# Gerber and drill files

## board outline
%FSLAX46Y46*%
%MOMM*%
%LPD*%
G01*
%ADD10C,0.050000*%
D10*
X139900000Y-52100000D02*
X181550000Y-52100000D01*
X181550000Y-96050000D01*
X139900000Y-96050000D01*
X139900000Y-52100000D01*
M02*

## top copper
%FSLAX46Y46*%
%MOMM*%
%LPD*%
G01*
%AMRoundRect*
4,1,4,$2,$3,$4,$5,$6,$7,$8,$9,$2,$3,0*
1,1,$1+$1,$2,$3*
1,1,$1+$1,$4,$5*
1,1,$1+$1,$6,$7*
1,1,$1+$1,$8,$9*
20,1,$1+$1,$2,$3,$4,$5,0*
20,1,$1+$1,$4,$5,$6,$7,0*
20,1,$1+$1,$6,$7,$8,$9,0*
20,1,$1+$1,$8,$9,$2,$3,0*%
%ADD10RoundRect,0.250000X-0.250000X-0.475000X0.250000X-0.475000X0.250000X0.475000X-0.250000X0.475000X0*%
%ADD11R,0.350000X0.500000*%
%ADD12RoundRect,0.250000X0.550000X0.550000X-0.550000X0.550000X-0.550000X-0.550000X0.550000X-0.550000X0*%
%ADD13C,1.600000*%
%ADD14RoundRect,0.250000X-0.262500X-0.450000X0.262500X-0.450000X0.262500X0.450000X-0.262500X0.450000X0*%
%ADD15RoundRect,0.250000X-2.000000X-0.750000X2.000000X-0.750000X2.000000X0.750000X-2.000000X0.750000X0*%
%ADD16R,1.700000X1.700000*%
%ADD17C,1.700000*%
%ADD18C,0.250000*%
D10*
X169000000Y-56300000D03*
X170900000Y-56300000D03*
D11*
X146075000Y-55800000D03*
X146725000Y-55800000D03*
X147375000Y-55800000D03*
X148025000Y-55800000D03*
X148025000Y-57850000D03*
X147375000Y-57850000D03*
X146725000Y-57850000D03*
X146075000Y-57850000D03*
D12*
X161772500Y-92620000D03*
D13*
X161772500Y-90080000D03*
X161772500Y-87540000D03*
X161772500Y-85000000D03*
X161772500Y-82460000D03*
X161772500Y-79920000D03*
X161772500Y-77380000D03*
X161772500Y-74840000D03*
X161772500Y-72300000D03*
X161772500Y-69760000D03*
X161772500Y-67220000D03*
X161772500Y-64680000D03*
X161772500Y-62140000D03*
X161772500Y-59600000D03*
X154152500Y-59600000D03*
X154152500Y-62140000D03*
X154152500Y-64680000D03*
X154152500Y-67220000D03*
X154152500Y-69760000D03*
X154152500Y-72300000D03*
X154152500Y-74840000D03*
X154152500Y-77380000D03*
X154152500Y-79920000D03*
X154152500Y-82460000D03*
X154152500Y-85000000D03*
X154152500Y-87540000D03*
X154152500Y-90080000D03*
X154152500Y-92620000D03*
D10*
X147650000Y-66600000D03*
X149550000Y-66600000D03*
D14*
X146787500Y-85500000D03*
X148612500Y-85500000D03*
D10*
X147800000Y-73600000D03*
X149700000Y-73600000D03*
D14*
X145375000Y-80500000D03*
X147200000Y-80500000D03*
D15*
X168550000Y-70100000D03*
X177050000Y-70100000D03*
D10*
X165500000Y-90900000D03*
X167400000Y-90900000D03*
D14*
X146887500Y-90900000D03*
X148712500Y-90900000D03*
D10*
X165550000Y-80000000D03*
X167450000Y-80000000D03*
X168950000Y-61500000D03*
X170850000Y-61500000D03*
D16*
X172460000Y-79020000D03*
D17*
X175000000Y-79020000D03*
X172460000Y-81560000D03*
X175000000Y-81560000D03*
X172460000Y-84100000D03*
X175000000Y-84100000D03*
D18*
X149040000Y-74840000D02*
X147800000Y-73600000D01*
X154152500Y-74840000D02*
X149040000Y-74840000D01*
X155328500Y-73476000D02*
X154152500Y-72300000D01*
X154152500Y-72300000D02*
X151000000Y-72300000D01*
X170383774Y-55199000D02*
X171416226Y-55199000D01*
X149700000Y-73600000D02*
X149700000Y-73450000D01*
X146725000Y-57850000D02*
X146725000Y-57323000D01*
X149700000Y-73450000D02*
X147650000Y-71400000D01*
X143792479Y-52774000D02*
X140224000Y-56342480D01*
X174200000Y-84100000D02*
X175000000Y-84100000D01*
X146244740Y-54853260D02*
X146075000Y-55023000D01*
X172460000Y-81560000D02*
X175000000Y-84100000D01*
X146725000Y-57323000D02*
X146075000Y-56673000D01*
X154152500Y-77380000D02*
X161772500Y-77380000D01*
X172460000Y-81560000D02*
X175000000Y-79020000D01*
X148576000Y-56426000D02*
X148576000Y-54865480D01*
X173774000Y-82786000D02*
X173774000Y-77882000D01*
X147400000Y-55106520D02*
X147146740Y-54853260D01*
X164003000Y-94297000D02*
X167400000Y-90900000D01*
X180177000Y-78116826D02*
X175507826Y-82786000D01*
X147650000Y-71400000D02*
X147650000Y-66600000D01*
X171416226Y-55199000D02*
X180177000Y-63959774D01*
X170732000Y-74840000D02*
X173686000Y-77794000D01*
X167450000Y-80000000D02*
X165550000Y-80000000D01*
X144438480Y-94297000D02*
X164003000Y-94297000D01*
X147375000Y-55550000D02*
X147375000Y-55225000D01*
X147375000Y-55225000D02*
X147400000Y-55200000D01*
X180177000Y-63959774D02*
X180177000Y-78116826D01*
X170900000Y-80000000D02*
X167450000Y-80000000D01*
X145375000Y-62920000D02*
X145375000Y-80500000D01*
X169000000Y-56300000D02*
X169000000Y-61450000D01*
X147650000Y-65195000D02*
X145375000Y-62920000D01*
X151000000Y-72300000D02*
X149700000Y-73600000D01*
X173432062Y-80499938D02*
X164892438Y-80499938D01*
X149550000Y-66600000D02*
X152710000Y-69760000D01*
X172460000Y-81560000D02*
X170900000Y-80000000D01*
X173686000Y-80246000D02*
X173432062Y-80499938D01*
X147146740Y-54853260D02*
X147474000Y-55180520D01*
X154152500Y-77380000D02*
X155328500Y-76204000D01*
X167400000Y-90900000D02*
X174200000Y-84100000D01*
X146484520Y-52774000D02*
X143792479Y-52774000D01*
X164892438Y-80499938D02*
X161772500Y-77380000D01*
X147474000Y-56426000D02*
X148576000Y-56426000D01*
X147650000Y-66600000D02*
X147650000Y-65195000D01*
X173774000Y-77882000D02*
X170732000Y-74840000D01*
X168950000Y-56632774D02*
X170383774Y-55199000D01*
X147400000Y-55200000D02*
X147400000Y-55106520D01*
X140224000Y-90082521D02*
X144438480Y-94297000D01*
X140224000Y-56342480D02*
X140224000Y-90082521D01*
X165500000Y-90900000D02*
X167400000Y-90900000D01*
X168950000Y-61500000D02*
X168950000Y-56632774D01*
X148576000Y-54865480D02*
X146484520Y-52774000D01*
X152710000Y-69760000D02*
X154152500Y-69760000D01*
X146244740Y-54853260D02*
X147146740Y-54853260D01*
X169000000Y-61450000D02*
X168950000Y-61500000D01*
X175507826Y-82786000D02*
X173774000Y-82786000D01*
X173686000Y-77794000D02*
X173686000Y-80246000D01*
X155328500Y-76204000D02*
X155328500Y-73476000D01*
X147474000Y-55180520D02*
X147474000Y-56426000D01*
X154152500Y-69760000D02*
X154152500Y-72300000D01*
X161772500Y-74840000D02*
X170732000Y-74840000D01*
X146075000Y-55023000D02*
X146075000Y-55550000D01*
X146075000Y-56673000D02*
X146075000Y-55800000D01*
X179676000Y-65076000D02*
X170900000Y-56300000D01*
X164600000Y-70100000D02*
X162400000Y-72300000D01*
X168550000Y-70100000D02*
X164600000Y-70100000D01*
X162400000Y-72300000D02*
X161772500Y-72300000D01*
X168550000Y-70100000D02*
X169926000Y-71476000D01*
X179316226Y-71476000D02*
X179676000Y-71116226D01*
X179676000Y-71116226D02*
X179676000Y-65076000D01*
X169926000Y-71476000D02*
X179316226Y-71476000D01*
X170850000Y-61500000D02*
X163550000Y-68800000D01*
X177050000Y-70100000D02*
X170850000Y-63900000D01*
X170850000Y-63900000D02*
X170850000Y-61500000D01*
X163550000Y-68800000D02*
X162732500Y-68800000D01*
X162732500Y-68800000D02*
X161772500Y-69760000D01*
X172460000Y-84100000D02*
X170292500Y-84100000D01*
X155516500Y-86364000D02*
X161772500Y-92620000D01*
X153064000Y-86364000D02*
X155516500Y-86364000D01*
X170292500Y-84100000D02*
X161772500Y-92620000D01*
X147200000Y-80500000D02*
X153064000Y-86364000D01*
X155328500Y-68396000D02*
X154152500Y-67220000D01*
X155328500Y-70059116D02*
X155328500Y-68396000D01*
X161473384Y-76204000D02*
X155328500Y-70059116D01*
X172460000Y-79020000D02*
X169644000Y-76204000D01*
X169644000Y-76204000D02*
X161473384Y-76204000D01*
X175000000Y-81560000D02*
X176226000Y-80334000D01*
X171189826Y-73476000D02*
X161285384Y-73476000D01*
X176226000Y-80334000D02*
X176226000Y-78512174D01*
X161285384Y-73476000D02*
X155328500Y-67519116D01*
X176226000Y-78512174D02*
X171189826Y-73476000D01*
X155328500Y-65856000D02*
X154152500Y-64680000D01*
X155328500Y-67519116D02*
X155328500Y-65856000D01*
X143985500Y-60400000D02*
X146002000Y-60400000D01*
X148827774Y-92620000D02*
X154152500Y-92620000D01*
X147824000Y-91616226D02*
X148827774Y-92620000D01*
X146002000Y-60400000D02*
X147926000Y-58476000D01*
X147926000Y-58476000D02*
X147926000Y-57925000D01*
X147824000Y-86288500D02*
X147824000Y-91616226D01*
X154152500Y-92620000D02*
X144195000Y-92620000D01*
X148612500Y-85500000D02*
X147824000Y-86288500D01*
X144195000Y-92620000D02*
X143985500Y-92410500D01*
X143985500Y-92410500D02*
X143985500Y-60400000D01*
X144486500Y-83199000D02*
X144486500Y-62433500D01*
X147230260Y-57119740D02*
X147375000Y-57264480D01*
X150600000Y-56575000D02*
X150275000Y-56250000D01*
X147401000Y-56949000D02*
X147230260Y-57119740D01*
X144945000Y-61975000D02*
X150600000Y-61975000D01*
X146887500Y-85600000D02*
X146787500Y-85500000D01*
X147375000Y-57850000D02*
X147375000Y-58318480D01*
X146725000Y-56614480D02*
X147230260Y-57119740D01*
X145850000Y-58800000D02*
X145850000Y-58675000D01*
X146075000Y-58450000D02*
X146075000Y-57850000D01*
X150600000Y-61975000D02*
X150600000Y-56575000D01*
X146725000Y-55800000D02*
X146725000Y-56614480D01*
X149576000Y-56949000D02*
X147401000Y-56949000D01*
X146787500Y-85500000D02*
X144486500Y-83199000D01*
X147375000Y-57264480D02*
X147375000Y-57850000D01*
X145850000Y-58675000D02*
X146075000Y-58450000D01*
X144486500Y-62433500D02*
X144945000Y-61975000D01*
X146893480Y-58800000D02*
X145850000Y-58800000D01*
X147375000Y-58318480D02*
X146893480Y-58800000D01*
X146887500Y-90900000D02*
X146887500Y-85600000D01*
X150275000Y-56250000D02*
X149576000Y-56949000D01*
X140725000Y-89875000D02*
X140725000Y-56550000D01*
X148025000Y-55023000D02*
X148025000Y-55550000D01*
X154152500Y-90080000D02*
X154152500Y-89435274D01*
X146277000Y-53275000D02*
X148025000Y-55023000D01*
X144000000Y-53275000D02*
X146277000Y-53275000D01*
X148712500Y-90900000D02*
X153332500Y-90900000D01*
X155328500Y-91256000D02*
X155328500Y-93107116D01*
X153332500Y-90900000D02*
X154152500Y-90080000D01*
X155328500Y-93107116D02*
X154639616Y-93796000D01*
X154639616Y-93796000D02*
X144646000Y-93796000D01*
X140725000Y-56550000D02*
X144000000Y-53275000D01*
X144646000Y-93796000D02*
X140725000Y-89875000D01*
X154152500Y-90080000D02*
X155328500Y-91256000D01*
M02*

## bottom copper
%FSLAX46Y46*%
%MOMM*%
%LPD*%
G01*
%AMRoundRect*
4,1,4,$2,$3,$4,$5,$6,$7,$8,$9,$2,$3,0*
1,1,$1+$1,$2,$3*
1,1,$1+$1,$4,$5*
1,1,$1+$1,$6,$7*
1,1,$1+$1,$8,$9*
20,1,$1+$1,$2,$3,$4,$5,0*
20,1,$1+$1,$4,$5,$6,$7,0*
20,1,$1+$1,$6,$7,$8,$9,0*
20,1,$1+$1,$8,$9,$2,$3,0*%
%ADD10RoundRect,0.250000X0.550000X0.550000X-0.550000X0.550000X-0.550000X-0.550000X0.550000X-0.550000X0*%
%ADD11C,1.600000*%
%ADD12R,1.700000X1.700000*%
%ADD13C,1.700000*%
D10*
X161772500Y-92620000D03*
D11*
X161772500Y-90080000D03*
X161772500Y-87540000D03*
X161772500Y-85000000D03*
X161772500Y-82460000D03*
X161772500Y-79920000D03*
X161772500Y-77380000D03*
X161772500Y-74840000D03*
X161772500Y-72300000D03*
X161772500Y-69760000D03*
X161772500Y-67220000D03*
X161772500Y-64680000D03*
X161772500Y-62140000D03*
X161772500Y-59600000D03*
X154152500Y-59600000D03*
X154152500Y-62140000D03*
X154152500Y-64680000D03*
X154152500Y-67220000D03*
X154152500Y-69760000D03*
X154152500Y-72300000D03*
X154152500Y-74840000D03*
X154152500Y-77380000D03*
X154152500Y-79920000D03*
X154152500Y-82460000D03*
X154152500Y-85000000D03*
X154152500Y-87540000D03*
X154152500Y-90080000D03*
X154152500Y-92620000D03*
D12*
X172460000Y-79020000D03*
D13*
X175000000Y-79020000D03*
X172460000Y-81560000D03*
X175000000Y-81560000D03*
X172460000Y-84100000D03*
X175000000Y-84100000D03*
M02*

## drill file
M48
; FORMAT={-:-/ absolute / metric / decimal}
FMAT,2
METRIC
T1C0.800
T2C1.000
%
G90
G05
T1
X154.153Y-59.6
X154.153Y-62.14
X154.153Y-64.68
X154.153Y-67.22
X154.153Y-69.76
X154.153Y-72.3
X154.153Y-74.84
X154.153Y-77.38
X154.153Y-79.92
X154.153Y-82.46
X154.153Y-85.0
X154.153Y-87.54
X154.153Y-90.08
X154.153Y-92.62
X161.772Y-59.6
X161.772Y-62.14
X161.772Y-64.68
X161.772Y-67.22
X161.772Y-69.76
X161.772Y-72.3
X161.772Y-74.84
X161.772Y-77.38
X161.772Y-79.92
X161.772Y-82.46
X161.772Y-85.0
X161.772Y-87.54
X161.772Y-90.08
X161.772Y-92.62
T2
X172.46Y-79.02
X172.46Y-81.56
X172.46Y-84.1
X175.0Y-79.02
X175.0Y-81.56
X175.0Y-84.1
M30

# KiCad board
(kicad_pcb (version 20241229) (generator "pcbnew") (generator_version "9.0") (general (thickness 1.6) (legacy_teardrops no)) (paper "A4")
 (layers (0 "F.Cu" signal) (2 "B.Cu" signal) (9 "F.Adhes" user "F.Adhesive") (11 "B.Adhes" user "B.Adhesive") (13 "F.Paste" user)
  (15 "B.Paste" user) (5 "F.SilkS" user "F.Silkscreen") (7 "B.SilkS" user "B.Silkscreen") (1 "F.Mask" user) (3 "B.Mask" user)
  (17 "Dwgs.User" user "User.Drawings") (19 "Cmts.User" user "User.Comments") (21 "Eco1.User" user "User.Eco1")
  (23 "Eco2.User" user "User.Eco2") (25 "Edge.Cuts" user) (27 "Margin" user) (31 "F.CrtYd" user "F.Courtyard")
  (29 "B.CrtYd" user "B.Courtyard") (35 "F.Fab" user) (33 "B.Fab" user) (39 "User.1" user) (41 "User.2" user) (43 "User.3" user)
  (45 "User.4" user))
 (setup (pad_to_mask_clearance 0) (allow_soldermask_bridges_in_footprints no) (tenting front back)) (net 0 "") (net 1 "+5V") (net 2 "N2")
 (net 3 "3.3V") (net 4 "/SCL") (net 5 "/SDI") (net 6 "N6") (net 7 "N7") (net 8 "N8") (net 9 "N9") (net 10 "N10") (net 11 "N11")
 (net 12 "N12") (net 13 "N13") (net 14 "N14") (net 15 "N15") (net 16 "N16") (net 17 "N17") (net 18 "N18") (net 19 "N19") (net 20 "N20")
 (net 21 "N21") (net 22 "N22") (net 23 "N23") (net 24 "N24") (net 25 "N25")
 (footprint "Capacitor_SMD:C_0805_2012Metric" (layer "F.Cu") (at 169.95 56.3)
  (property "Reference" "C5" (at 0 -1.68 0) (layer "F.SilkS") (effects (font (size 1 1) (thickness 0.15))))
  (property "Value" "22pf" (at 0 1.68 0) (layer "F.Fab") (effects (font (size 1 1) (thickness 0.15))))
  (pad "1" smd roundrect (at -0.95 0) (size 1 1.45) (layers "F.Cu" "F.Mask" "F.Paste") (roundrect_rratio 0.25) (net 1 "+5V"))
  (pad "2" smd roundrect (at 0.95 0) (size 1 1.45) (layers "F.Cu" "F.Mask" "F.Paste") (roundrect_rratio 0.25) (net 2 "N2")))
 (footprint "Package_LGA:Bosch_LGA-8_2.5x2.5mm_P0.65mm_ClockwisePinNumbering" (layer "F.Cu") (at 147.05 56.825)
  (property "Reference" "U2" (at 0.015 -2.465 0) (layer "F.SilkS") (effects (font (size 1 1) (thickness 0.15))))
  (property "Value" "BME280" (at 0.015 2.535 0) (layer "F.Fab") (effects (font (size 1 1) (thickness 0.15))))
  (pad "1" smd rect (at -0.975 -1.025 90) (size 0.5 0.35) (layers "F.Cu" "F.Mask" "F.Paste") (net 1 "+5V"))
  (pad "2" smd rect (at -0.325 -1.025 90) (size 0.5 0.35) (layers "F.Cu" "F.Mask" "F.Paste") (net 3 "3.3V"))
  (pad "3" smd rect (at 0.325 -1.025 90) (size 0.5 0.35) (layers "F.Cu" "F.Mask" "F.Paste") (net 1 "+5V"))
  (pad "4" smd rect (at 0.975 -1.025 90) (size 0.5 0.35) (layers "F.Cu" "F.Mask" "F.Paste") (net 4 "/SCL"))
  (pad "5" smd rect (at 0.975 1.025 90) (size 0.5 0.35) (layers "F.Cu" "F.Mask" "F.Paste") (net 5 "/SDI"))
  (pad "6" smd rect (at 0.325 1.025 90) (size 0.5 0.35) (layers "F.Cu" "F.Mask" "F.Paste") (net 3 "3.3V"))
  (pad "7" smd rect (at -0.325 1.025 90) (size 0.5 0.35) (layers "F.Cu" "F.Mask" "F.Paste") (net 1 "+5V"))
  (pad "8" smd rect (at -0.975 1.025 90) (size 0.5 0.35) (layers "F.Cu" "F.Mask" "F.Paste") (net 3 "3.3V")))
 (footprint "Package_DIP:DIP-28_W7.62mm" (layer "F.Cu") (at 161.7725 92.62 180)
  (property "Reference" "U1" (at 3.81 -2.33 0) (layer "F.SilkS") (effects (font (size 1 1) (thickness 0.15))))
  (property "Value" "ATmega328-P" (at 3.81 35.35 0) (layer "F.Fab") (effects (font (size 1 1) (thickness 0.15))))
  (pad "1" thru_hole roundrect (at 0 0 180) (size 1.6 1.6) (drill 0.8) (layers "*.Cu" "*.Mask") (remove_unused_layers no)
   (roundrect_rratio 0.15625) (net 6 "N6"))
  (pad "2" thru_hole circle (at 0 2.54 180) (size 1.6 1.6) (drill 0.8) (layers "*.Cu" "*.Mask") (remove_unused_layers no) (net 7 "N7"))
  (pad "3" thru_hole circle (at 0 5.08 180) (size 1.6 1.6) (drill 0.8) (layers "*.Cu" "*.Mask") (remove_unused_layers no) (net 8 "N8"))
  (pad "4" thru_hole circle (at 0 7.62 180) (size 1.6 1.6) (drill 0.8) (layers "*.Cu" "*.Mask") (remove_unused_layers no) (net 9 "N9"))
  (pad "5" thru_hole circle (at 0 10.16 180) (size 1.6 1.6) (drill 0.8) (layers "*.Cu" "*.Mask") (remove_unused_layers no) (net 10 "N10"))
  (pad "6" thru_hole circle (at 0 12.7 180) (size 1.6 1.6) (drill 0.8) (layers "*.Cu" "*.Mask") (remove_unused_layers no) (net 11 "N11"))
  (pad "7" thru_hole circle (at 0 15.24 180) (size 1.6 1.6) (drill 0.8) (layers "*.Cu" "*.Mask") (remove_unused_layers no) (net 1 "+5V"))
  (pad "8" thru_hole circle (at 0 17.78 180) (size 1.6 1.6) (drill 0.8) (layers "*.Cu" "*.Mask") (remove_unused_layers no) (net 1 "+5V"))
  (pad "9" thru_hole circle (at 0 20.32 180) (size 1.6 1.6) (drill 0.8) (layers "*.Cu" "*.Mask") (remove_unused_layers no) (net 2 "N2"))
  (pad "10" thru_hole circle (at 0 22.86 180) (size 1.6 1.6) (drill 0.8) (layers "*.Cu" "*.Mask") (remove_unused_layers no) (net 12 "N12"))
  (pad "11" thru_hole circle (at 0 25.4 180) (size 1.6 1.6) (drill 0.8) (layers "*.Cu" "*.Mask") (remove_unused_layers no) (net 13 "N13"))
  (pad "12" thru_hole circle (at 0 27.94 180) (size 1.6 1.6) (drill 0.8) (layers "*.Cu" "*.Mask") (remove_unused_layers no) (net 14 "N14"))
  (pad "13" thru_hole circle (at 0 30.48 180) (size 1.6 1.6) (drill 0.8) (layers "*.Cu" "*.Mask") (remove_unused_layers no) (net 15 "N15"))
  (pad "14" thru_hole circle (at 0 33.02 180) (size 1.6 1.6) (drill 0.8) (layers "*.Cu" "*.Mask") (remove_unused_layers no) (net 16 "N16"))
  (pad "15" thru_hole circle (at 7.62 33.02 180) (size 1.6 1.6) (drill 0.8) (layers "*.Cu" "*.Mask") (remove_unused_layers no)
   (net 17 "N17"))
  (pad "16" thru_hole circle (at 7.62 30.48 180) (size 1.6 1.6) (drill 0.8) (layers "*.Cu" "*.Mask") (remove_unused_layers no)
   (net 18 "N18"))
  (pad "17" thru_hole circle (at 7.62 27.94 180) (size 1.6 1.6) (drill 0.8) (layers "*.Cu" "*.Mask") (remove_unused_layers no)
   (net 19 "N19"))
  (pad "18" thru_hole circle (at 7.62 25.4 180) (size 1.6 1.6) (drill 0.8) (layers "*.Cu" "*.Mask") (remove_unused_layers no) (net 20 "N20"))
  (pad "19" thru_hole circle (at 7.62 22.86 180) (size 1.6 1.6) (drill 0.8) (layers "*.Cu" "*.Mask") (remove_unused_layers no) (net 1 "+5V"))
  (pad "20" thru_hole circle (at 7.62 20.32 180) (size 1.6 1.6) (drill 0.8) (layers "*.Cu" "*.Mask") (remove_unused_layers no) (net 1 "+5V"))
  (pad "21" thru_hole circle (at 7.62 17.78 180) (size 1.6 1.6) (drill 0.8) (layers "*.Cu" "*.Mask") (remove_unused_layers no)
   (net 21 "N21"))
  (pad "22" thru_hole circle (at 7.62 15.24 180) (size 1.6 1.6) (drill 0.8) (layers "*.Cu" "*.Mask") (remove_unused_layers no) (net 1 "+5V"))
  (pad "23" thru_hole circle (at 7.62 12.7 180) (size 1.6 1.6) (drill 0.8) (layers "*.Cu" "*.Mask") (remove_unused_layers no) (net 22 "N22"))
  (pad "24" thru_hole circle (at 7.62 10.16 180) (size 1.6 1.6) (drill 0.8) (layers "*.Cu" "*.Mask") (remove_unused_layers no)
   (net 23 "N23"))
  (pad "25" thru_hole circle (at 7.62 7.62 180) (size 1.6 1.6) (drill 0.8) (layers "*.Cu" "*.Mask") (remove_unused_layers no) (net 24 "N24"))
  (pad "26" thru_hole circle (at 7.62 5.08 180) (size 1.6 1.6) (drill 0.8) (layers "*.Cu" "*.Mask") (remove_unused_layers no) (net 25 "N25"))
  (pad "27" thru_hole circle (at 7.62 2.54 180) (size 1.6 1.6) (drill 0.8) (layers "*.Cu" "*.Mask") (remove_unused_layers no) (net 4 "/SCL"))
  (pad "28" thru_hole circle (at 7.62 0 180) (size 1.6 1.6) (drill 0.8) (layers "*.Cu" "*.Mask") (remove_unused_layers no) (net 5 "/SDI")))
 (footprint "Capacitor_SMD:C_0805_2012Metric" (layer "F.Cu") (at 148.6 66.6)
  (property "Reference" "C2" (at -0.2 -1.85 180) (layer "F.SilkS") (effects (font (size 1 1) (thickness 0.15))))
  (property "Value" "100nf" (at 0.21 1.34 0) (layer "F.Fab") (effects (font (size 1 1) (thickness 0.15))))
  (pad "1" smd roundrect (at -0.95 0) (size 1 1.45) (layers "F.Cu" "F.Mask" "F.Paste") (roundrect_rratio 0.25) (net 1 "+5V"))
  (pad "2" smd roundrect (at 0.95 0) (size 1 1.45) (layers "F.Cu" "F.Mask" "F.Paste") (roundrect_rratio 0.25) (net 1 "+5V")))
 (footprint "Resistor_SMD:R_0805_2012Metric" (layer "F.Cu") (at 147.7 85.5)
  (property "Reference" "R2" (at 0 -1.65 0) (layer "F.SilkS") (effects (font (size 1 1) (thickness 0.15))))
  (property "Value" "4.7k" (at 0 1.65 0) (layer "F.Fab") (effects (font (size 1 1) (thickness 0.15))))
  (pad "1" smd roundrect (at -0.9125 0) (size 1.025 1.4) (layers "F.Cu" "F.Mask" "F.Paste") (roundrect_rratio 0.243902) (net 3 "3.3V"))
  (pad "2" smd roundrect (at 0.9125 0) (size 1.025 1.4) (layers "F.Cu" "F.Mask" "F.Paste") (roundrect_rratio 0.243902) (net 5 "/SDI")))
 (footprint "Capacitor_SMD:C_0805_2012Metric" (layer "F.Cu") (at 148.75 73.6)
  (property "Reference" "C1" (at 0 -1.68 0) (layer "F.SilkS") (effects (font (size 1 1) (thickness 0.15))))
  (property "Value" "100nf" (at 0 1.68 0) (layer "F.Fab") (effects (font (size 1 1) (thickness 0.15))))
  (pad "1" smd roundrect (at -0.95 0) (size 1 1.45) (layers "F.Cu" "F.Mask" "F.Paste") (roundrect_rratio 0.25) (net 21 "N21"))
  (pad "2" smd roundrect (at 0.95 0) (size 1 1.45) (layers "F.Cu" "F.Mask" "F.Paste") (roundrect_rratio 0.25) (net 1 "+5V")))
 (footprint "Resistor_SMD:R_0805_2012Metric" (layer "F.Cu") (at 146.2875 80.5)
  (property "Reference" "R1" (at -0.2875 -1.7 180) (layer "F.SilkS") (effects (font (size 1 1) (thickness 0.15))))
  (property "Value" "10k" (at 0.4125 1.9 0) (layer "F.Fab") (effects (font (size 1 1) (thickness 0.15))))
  (pad "1" smd roundrect (at -0.9125 0) (size 1.025 1.4) (layers "F.Cu" "F.Mask" "F.Paste") (roundrect_rratio 0.243902) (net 1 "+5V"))
  (pad "2" smd roundrect (at 0.9125 0) (size 1.025 1.4) (layers "F.Cu" "F.Mask" "F.Paste") (roundrect_rratio 0.243902) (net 6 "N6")))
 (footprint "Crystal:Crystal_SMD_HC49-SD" (layer "F.Cu") (at 172.8 70.1)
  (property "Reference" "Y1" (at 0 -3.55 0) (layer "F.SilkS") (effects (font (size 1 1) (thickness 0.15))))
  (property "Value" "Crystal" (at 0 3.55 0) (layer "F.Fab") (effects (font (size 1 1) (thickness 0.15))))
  (pad "1" smd roundrect (at -4.25 0) (size 4.5 2) (layers "F.Cu" "F.Mask" "F.Paste") (roundrect_rratio 0.125) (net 2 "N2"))
  (pad "2" smd roundrect (at 4.25 0) (size 4.5 2) (layers "F.Cu" "F.Mask" "F.Paste") (roundrect_rratio 0.125) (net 12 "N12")))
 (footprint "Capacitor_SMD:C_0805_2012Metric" (layer "F.Cu") (at 166.45 90.9)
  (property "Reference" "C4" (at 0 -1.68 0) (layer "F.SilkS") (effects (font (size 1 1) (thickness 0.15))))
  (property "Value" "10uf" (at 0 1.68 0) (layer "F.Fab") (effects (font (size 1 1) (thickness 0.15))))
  (pad "1" smd roundrect (at -0.95 0) (size 1 1.45) (layers "F.Cu" "F.Mask" "F.Paste") (roundrect_rratio 0.25) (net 1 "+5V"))
  (pad "2" smd roundrect (at 0.95 0) (size 1 1.45) (layers "F.Cu" "F.Mask" "F.Paste") (roundrect_rratio 0.25) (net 1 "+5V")))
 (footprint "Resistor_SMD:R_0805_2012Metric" (layer "F.Cu") (at 147.8 90.9)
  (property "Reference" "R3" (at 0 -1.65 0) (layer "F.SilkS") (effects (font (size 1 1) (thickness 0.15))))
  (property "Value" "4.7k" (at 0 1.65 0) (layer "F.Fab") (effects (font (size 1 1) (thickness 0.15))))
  (pad "1" smd roundrect (at -0.9125 0) (size 1.025 1.4) (layers "F.Cu" "F.Mask" "F.Paste") (roundrect_rratio 0.243902) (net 3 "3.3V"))
  (pad "2" smd roundrect (at 0.9125 0) (size 1.025 1.4) (layers "F.Cu" "F.Mask" "F.Paste") (roundrect_rratio 0.243902) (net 4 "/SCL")))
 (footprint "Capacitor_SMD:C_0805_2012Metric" (layer "F.Cu") (at 166.5 80)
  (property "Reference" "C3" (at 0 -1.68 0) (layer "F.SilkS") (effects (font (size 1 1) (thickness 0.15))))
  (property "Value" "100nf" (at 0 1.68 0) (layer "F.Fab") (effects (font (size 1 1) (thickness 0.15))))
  (pad "1" smd roundrect (at -0.95 0) (size 1 1.45) (layers "F.Cu" "F.Mask" "F.Paste") (roundrect_rratio 0.25) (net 1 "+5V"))
  (pad "2" smd roundrect (at 0.95 0) (size 1 1.45) (layers "F.Cu" "F.Mask" "F.Paste") (roundrect_rratio 0.25) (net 1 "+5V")))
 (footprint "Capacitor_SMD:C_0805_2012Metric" (layer "F.Cu") (at 169.9 61.5)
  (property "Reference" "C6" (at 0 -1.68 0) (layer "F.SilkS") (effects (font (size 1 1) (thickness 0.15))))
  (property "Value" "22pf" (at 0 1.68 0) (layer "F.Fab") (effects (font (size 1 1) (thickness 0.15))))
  (pad "1" smd roundrect (at -0.95 0) (size 1 1.45) (layers "F.Cu" "F.Mask" "F.Paste") (roundrect_rratio 0.25) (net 1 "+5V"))
  (pad "2" smd roundrect (at 0.95 0) (size 1 1.45) (layers "F.Cu" "F.Mask" "F.Paste") (roundrect_rratio 0.25) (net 12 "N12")))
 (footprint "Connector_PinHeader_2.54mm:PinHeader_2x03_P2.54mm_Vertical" (layer "F.Cu") (at 172.46 79.02)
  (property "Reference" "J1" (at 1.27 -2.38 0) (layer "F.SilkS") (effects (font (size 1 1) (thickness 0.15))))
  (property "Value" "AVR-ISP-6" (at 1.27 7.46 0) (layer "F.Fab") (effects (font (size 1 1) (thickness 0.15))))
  (pad "1" thru_hole rect (at 0 0) (size 1.7 1.7) (drill 1) (layers "*.Cu" "*.Mask") (remove_unused_layers no) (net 20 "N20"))
  (pad "2" thru_hole circle (at 2.54 0) (size 1.7 1.7) (drill 1) (layers "*.Cu" "*.Mask") (remove_unused_layers no) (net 1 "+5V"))
  (pad "3" thru_hole circle (at 0 2.54) (size 1.7 1.7) (drill 1) (layers "*.Cu" "*.Mask") (remove_unused_layers no) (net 1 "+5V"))
  (pad "4" thru_hole circle (at 2.54 2.54) (size 1.7 1.7) (drill 1) (layers "*.Cu" "*.Mask") (remove_unused_layers no) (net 19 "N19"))
  (pad "5" thru_hole circle (at 0 5.08) (size 1.7 1.7) (drill 1) (layers "*.Cu" "*.Mask") (remove_unused_layers no) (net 6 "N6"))
  (pad "6" thru_hole circle (at 2.54 5.08) (size 1.7 1.7) (drill 1) (layers "*.Cu" "*.Mask") (remove_unused_layers no) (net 1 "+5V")))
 (gr_rect (start 139.9 52.1) (end 181.55 96.05) (stroke (width 0.05) (type default)) (fill no) (layer "Edge.Cuts"))
 (segment (start 149.04 74.84) (end 147.8 73.6) (width 0.25) (layer "F.Cu") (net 21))
 (segment (start 154.1525 74.84) (end 149.04 74.84) (width 0.25) (layer "F.Cu") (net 21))
 (segment (start 155.3285 73.476) (end 154.1525 72.3) (width 0.25) (layer "F.Cu") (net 1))
 (segment (start 154.1525 72.3) (end 151 72.3) (width 0.25) (layer "F.Cu") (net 1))
 (segment (start 170.383774 55.199) (end 171.416226 55.199) (width 0.25) (layer "F.Cu") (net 1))
 (segment (start 149.7 73.6) (end 149.7 73.45) (width 0.25) (layer "F.Cu") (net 1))
 (segment (start 146.725 57.85) (end 146.725 57.323) (width 0.25) (layer "F.Cu") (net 1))
 (segment (start 149.7 73.45) (end 147.65 71.4) (width 0.25) (layer "F.Cu") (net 1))
 (segment (start 143.792479 52.774) (end 140.224 56.34248) (width 0.25) (layer "F.Cu") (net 1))
 (segment (start 174.2 84.1) (end 175 84.1) (width 0.25) (layer "F.Cu") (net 1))
 (segment (start 146.24474 54.85326) (end 146.075 55.023) (width 0.25) (layer "F.Cu") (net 1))
 (segment (start 172.46 81.56) (end 175 84.1) (width 0.25) (layer "F.Cu") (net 1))
 (segment (start 146.725 57.323) (end 146.075 56.673) (width 0.25) (layer "F.Cu") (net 1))
 (segment (start 154.1525 77.38) (end 161.7725 77.38) (width 0.25) (layer "F.Cu") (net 1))
 (segment (start 172.46 81.56) (end 175 79.02) (width 0.25) (layer "F.Cu") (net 1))
 (segment (start 148.576 56.426) (end 148.576 54.86548) (width 0.25) (layer "F.Cu") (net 1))
 (segment (start 173.774 82.786) (end 173.774 77.882) (width 0.25) (layer "F.Cu") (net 1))
 (segment (start 147.4 55.10652) (end 147.14674 54.85326) (width 0.25) (layer "F.Cu") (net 1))
 (segment (start 164.003 94.297) (end 167.4 90.9) (width 0.25) (layer "F.Cu") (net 1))
 (segment (start 180.177 78.116826) (end 175.507826 82.786) (width 0.25) (layer "F.Cu") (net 1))
 (segment (start 147.65 71.4) (end 147.65 66.6) (width 0.25) (layer "F.Cu") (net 1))
 (segment (start 171.416226 55.199) (end 180.177 63.959774) (width 0.25) (layer "F.Cu") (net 1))
 (segment (start 170.732 74.84) (end 173.686 77.794) (width 0.25) (layer "F.Cu") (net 1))
 (segment (start 167.45 80) (end 165.55 80) (width 0.25) (layer "F.Cu") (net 1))
 (segment (start 144.43848 94.297) (end 164.003 94.297) (width 0.25) (layer "F.Cu") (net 1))
 (segment (start 147.375 55.55) (end 147.375 55.225) (width 0.25) (layer "F.Cu") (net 1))
 (segment (start 147.375 55.225) (end 147.4 55.2) (width 0.25) (layer "F.Cu") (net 1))
 (segment (start 180.177 63.959774) (end 180.177 78.116826) (width 0.25) (layer "F.Cu") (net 1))
 (segment (start 170.9 80) (end 167.45 80) (width 0.25) (layer "F.Cu") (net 1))
 (segment (start 145.375 62.92) (end 145.375 80.5) (width 0.25) (layer "F.Cu") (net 1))
 (segment (start 169 56.3) (end 169 61.45) (width 0.25) (layer "F.Cu") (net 1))
 (segment (start 147.65 65.195) (end 145.375 62.92) (width 0.25) (layer "F.Cu") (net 1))
 (segment (start 151 72.3) (end 149.7 73.6) (width 0.25) (layer "F.Cu") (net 1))
 (segment (start 173.432062 80.499938) (end 164.892438 80.499938) (width 0.25) (layer "F.Cu") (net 1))
 (segment (start 149.55 66.6) (end 152.71 69.76) (width 0.25) (layer "F.Cu") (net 1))
 (segment (start 172.46 81.56) (end 170.9 80) (width 0.25) (layer "F.Cu") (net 1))
 (segment (start 173.686 80.246) (end 173.432062 80.499938) (width 0.25) (layer "F.Cu") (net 1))
 (segment (start 147.14674 54.85326) (end 147.474 55.18052) (width 0.25) (layer "F.Cu") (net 1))
 (segment (start 154.1525 77.38) (end 155.3285 76.204) (width 0.25) (layer "F.Cu") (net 1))
 (segment (start 167.4 90.9) (end 174.2 84.1) (width 0.25) (layer "F.Cu") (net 1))
 (segment (start 146.48452 52.774) (end 143.792479 52.774) (width 0.25) (layer "F.Cu") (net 1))
 (segment (start 164.892438 80.499938) (end 161.7725 77.38) (width 0.25) (layer "F.Cu") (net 1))
 (segment (start 147.474 56.426) (end 148.576 56.426) (width 0.25) (layer "F.Cu") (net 1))
 (segment (start 147.65 66.6) (end 147.65 65.195) (width 0.25) (layer "F.Cu") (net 1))
 (segment (start 173.774 77.882) (end 170.732 74.84) (width 0.25) (layer "F.Cu") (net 1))
 (segment (start 168.95 56.632774) (end 170.383774 55.199) (width 0.25) (layer "F.Cu") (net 1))
 (segment (start 147.4 55.2) (end 147.4 55.10652) (width 0.25) (layer "F.Cu") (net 1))
 (segment (start 140.224 90.082521) (end 144.43848 94.297) (width 0.25) (layer "F.Cu") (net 1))
 (segment (start 140.224 56.34248) (end 140.224 90.082521) (width 0.25) (layer "F.Cu") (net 1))
 (segment (start 165.5 90.9) (end 167.4 90.9) (width 0.25) (layer "F.Cu") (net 1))
 (segment (start 168.95 61.5) (end 168.95 56.632774) (width 0.25) (layer "F.Cu") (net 1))
 (segment (start 148.576 54.86548) (end 146.48452 52.774) (width 0.25) (layer "F.Cu") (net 1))
 (segment (start 152.71 69.76) (end 154.1525 69.76) (width 0.25) (layer "F.Cu") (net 1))
 (segment (start 146.24474 54.85326) (end 147.14674 54.85326) (width 0.25) (layer "F.Cu") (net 1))
 (segment (start 169 61.45) (end 168.95 61.5) (width 0.25) (layer "F.Cu") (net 1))
 (segment (start 175.507826 82.786) (end 173.774 82.786) (width 0.25) (layer "F.Cu") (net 1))
 (segment (start 173.686 77.794) (end 173.686 80.246) (width 0.25) (layer "F.Cu") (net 1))
 (segment (start 155.3285 76.204) (end 155.3285 73.476) (width 0.25) (layer "F.Cu") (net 1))
 (segment (start 147.474 55.18052) (end 147.474 56.426) (width 0.25) (layer "F.Cu") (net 1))
 (segment (start 154.1525 69.76) (end 154.1525 72.3) (width 0.25) (layer "F.Cu") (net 1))
 (segment (start 161.7725 74.84) (end 170.732 74.84) (width 0.25) (layer "F.Cu") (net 1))
 (segment (start 146.075 55.023) (end 146.075 55.55) (width 0.25) (layer "F.Cu") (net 1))
 (segment (start 146.075 56.673) (end 146.075 55.8) (width 0.25) (layer "F.Cu") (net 1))
 (segment (start 179.676 65.076) (end 170.9 56.3) (width 0.25) (layer "F.Cu") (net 2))
 (segment (start 164.6 70.1) (end 162.4 72.3) (width 0.25) (layer "F.Cu") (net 2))
 (segment (start 168.55 70.1) (end 164.6 70.1) (width 0.25) (layer "F.Cu") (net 2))
 (segment (start 162.4 72.3) (end 161.7725 72.3) (width 0.25) (layer "F.Cu") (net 2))
 (segment (start 168.55 70.1) (end 169.926 71.476) (width 0.25) (layer "F.Cu") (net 2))
 (segment (start 179.316226 71.476) (end 179.676 71.116226) (width 0.25) (layer "F.Cu") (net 2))
 (segment (start 179.676 71.116226) (end 179.676 65.076) (width 0.25) (layer "F.Cu") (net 2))
 (segment (start 169.926 71.476) (end 179.316226 71.476) (width 0.25) (layer "F.Cu") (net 2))
 (segment (start 170.85 61.5) (end 163.55 68.8) (width 0.25) (layer "F.Cu") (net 12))
 (segment (start 177.05 70.1) (end 170.85 63.9) (width 0.25) (layer "F.Cu") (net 12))
 (segment (start 170.85 63.9) (end 170.85 61.5) (width 0.25) (layer "F.Cu") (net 12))
 (segment (start 163.55 68.8) (end 162.7325 68.8) (width 0.25) (layer "F.Cu") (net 12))
 (segment (start 162.7325 68.8) (end 161.7725 69.76) (width 0.25) (layer "F.Cu") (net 12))
 (segment (start 172.46 84.1) (end 170.2925 84.1) (width 0.25) (layer "F.Cu") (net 6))
 (segment (start 155.5165 86.364) (end 161.7725 92.62) (width 0.25) (layer "F.Cu") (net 6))
 (segment (start 153.064 86.364) (end 155.5165 86.364) (width 0.25) (layer "F.Cu") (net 6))
 (segment (start 170.2925 84.1) (end 161.7725 92.62) (width 0.25) (layer "F.Cu") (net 6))
 (segment (start 147.2 80.5) (end 153.064 86.364) (width 0.25) (layer "F.Cu") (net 6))
 (segment (start 155.3285 68.396) (end 154.1525 67.22) (width 0.25) (layer "F.Cu") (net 20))
 (segment (start 155.3285 70.059116) (end 155.3285 68.396) (width 0.25) (layer "F.Cu") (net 20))
 (segment (start 161.473384 76.204) (end 155.3285 70.059116) (width 0.25) (layer "F.Cu") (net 20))
 (segment (start 172.46 79.02) (end 169.644 76.204) (width 0.25) (layer "F.Cu") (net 20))
 (segment (start 169.644 76.204) (end 161.473384 76.204) (width 0.25) (layer "F.Cu") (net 20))
 (segment (start 175 81.56) (end 176.226 80.334) (width 0.25) (layer "F.Cu") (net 19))
 (segment (start 171.189826 73.476) (end 161.285384 73.476) (width 0.25) (layer "F.Cu") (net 19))
 (segment (start 176.226 80.334) (end 176.226 78.512174) (width 0.25) (layer "F.Cu") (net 19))
 (segment (start 161.285384 73.476) (end 155.3285 67.519116) (width 0.25) (layer "F.Cu") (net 19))
 (segment (start 176.226 78.512174) (end 171.189826 73.476) (width 0.25) (layer "F.Cu") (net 19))
 (segment (start 155.3285 65.856) (end 154.1525 64.68) (width 0.25) (layer "F.Cu") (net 19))
 (segment (start 155.3285 67.519116) (end 155.3285 65.856) (width 0.25) (layer "F.Cu") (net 19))
 (segment (start 143.9855 60.4) (end 146.002 60.4) (width 0.25) (layer "F.Cu") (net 5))
 (segment (start 148.827774 92.62) (end 154.1525 92.62) (width 0.25) (layer "F.Cu") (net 5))
 (segment (start 147.824 91.616226) (end 148.827774 92.62) (width 0.25) (layer "F.Cu") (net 5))
 (segment (start 146.002 60.4) (end 147.926 58.476) (width 0.25) (layer "F.Cu") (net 5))
 (segment (start 147.926 58.476) (end 147.926 57.925) (width 0.25) (layer "F.Cu") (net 5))
 (segment (start 147.824 86.2885) (end 147.824 91.616226) (width 0.25) (layer "F.Cu") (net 5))
 (segment (start 154.1525 92.62) (end 144.195 92.62) (width 0.25) (layer "F.Cu") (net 5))
 (segment (start 148.6125 85.5) (end 147.824 86.2885) (width 0.25) (layer "F.Cu") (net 5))
 (segment (start 144.195 92.62) (end 143.9855 92.4105) (width 0.25) (layer "F.Cu") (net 5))
 (segment (start 143.9855 92.4105) (end 143.9855 60.4) (width 0.25) (layer "F.Cu") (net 5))
 (segment (start 144.4865 83.199) (end 144.4865 62.4335) (width 0.25) (layer "F.Cu") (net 3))
 (segment (start 147.23026 57.11974) (end 147.375 57.26448) (width 0.25) (layer "F.Cu") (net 3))
 (segment (start 150.6 56.575) (end 150.275 56.25) (width 0.25) (layer "F.Cu") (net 3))
 (segment (start 147.401 56.949) (end 147.23026 57.11974) (width 0.25) (layer "F.Cu") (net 3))
 (segment (start 144.945 61.975) (end 150.6 61.975) (width 0.25) (layer "F.Cu") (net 3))
 (segment (start 146.8875 85.6) (end 146.7875 85.5) (width 0.25) (layer "F.Cu") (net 3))
 (segment (start 147.375 57.85) (end 147.375 58.31848) (width 0.25) (layer "F.Cu") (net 3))
 (segment (start 146.725 56.61448) (end 147.23026 57.11974) (width 0.25) (layer "F.Cu") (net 3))
 (segment (start 145.85 58.8) (end 145.85 58.675) (width 0.25) (layer "F.Cu") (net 3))
 (segment (start 146.075 58.45) (end 146.075 57.85) (width 0.25) (layer "F.Cu") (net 3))
 (segment (start 150.6 61.975) (end 150.6 56.575) (width 0.25) (layer "F.Cu") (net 3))
 (segment (start 146.725 55.8) (end 146.725 56.61448) (width 0.25) (layer "F.Cu") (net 3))
 (segment (start 149.576 56.949) (end 147.401 56.949) (width 0.25) (layer "F.Cu") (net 3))
 (segment (start 146.7875 85.5) (end 144.4865 83.199) (width 0.25) (layer "F.Cu") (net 3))
 (segment (start 147.375 57.26448) (end 147.375 57.85) (width 0.25) (layer "F.Cu") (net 3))
 (segment (start 145.85 58.675) (end 146.075 58.45) (width 0.25) (layer "F.Cu") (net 3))
 (segment (start 144.4865 62.4335) (end 144.945 61.975) (width 0.25) (layer "F.Cu") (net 3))
 (segment (start 146.89348 58.8) (end 145.85 58.8) (width 0.25) (layer "F.Cu") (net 3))
 (segment (start 147.375 58.31848) (end 146.89348 58.8) (width 0.25) (layer "F.Cu") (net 3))
 (segment (start 146.8875 90.9) (end 146.8875 85.6) (width 0.25) (layer "F.Cu") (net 3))
 (segment (start 150.275 56.25) (end 149.576 56.949) (width 0.25) (layer "F.Cu") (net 3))
 (segment (start 140.725 89.875) (end 140.725 56.55) (width 0.25) (layer "F.Cu") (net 4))
 (segment (start 148.025 55.023) (end 148.025 55.55) (width 0.25) (layer "F.Cu") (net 4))
 (segment (start 154.1525 90.08) (end 154.1525 89.435274) (width 0.25) (layer "F.Cu") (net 4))
 (segment (start 146.277 53.275) (end 148.025 55.023) (width 0.25) (layer "F.Cu") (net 4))
 (segment (start 144 53.275) (end 146.277 53.275) (width 0.25) (layer "F.Cu") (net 4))
 (segment (start 148.7125 90.9) (end 153.3325 90.9) (width 0.25) (layer "F.Cu") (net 4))
 (segment (start 155.3285 91.256) (end 155.3285 93.107116) (width 0.25) (layer "F.Cu") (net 4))
 (segment (start 153.3325 90.9) (end 154.1525 90.08) (width 0.25) (layer "F.Cu") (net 4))
 (segment (start 155.3285 93.107116) (end 154.639616 93.796) (width 0.25) (layer "F.Cu") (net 4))
 (segment (start 154.639616 93.796) (end 144.646 93.796) (width 0.25) (layer "F.Cu") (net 4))
 (segment (start 140.725 56.55) (end 144 53.275) (width 0.25) (layer "F.Cu") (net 4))
 (segment (start 144.646 93.796) (end 140.725 89.875) (width 0.25) (layer "F.Cu") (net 4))
 (segment (start 154.1525 90.08) (end 155.3285 91.256) (width 0.25) (layer "F.Cu") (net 4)))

